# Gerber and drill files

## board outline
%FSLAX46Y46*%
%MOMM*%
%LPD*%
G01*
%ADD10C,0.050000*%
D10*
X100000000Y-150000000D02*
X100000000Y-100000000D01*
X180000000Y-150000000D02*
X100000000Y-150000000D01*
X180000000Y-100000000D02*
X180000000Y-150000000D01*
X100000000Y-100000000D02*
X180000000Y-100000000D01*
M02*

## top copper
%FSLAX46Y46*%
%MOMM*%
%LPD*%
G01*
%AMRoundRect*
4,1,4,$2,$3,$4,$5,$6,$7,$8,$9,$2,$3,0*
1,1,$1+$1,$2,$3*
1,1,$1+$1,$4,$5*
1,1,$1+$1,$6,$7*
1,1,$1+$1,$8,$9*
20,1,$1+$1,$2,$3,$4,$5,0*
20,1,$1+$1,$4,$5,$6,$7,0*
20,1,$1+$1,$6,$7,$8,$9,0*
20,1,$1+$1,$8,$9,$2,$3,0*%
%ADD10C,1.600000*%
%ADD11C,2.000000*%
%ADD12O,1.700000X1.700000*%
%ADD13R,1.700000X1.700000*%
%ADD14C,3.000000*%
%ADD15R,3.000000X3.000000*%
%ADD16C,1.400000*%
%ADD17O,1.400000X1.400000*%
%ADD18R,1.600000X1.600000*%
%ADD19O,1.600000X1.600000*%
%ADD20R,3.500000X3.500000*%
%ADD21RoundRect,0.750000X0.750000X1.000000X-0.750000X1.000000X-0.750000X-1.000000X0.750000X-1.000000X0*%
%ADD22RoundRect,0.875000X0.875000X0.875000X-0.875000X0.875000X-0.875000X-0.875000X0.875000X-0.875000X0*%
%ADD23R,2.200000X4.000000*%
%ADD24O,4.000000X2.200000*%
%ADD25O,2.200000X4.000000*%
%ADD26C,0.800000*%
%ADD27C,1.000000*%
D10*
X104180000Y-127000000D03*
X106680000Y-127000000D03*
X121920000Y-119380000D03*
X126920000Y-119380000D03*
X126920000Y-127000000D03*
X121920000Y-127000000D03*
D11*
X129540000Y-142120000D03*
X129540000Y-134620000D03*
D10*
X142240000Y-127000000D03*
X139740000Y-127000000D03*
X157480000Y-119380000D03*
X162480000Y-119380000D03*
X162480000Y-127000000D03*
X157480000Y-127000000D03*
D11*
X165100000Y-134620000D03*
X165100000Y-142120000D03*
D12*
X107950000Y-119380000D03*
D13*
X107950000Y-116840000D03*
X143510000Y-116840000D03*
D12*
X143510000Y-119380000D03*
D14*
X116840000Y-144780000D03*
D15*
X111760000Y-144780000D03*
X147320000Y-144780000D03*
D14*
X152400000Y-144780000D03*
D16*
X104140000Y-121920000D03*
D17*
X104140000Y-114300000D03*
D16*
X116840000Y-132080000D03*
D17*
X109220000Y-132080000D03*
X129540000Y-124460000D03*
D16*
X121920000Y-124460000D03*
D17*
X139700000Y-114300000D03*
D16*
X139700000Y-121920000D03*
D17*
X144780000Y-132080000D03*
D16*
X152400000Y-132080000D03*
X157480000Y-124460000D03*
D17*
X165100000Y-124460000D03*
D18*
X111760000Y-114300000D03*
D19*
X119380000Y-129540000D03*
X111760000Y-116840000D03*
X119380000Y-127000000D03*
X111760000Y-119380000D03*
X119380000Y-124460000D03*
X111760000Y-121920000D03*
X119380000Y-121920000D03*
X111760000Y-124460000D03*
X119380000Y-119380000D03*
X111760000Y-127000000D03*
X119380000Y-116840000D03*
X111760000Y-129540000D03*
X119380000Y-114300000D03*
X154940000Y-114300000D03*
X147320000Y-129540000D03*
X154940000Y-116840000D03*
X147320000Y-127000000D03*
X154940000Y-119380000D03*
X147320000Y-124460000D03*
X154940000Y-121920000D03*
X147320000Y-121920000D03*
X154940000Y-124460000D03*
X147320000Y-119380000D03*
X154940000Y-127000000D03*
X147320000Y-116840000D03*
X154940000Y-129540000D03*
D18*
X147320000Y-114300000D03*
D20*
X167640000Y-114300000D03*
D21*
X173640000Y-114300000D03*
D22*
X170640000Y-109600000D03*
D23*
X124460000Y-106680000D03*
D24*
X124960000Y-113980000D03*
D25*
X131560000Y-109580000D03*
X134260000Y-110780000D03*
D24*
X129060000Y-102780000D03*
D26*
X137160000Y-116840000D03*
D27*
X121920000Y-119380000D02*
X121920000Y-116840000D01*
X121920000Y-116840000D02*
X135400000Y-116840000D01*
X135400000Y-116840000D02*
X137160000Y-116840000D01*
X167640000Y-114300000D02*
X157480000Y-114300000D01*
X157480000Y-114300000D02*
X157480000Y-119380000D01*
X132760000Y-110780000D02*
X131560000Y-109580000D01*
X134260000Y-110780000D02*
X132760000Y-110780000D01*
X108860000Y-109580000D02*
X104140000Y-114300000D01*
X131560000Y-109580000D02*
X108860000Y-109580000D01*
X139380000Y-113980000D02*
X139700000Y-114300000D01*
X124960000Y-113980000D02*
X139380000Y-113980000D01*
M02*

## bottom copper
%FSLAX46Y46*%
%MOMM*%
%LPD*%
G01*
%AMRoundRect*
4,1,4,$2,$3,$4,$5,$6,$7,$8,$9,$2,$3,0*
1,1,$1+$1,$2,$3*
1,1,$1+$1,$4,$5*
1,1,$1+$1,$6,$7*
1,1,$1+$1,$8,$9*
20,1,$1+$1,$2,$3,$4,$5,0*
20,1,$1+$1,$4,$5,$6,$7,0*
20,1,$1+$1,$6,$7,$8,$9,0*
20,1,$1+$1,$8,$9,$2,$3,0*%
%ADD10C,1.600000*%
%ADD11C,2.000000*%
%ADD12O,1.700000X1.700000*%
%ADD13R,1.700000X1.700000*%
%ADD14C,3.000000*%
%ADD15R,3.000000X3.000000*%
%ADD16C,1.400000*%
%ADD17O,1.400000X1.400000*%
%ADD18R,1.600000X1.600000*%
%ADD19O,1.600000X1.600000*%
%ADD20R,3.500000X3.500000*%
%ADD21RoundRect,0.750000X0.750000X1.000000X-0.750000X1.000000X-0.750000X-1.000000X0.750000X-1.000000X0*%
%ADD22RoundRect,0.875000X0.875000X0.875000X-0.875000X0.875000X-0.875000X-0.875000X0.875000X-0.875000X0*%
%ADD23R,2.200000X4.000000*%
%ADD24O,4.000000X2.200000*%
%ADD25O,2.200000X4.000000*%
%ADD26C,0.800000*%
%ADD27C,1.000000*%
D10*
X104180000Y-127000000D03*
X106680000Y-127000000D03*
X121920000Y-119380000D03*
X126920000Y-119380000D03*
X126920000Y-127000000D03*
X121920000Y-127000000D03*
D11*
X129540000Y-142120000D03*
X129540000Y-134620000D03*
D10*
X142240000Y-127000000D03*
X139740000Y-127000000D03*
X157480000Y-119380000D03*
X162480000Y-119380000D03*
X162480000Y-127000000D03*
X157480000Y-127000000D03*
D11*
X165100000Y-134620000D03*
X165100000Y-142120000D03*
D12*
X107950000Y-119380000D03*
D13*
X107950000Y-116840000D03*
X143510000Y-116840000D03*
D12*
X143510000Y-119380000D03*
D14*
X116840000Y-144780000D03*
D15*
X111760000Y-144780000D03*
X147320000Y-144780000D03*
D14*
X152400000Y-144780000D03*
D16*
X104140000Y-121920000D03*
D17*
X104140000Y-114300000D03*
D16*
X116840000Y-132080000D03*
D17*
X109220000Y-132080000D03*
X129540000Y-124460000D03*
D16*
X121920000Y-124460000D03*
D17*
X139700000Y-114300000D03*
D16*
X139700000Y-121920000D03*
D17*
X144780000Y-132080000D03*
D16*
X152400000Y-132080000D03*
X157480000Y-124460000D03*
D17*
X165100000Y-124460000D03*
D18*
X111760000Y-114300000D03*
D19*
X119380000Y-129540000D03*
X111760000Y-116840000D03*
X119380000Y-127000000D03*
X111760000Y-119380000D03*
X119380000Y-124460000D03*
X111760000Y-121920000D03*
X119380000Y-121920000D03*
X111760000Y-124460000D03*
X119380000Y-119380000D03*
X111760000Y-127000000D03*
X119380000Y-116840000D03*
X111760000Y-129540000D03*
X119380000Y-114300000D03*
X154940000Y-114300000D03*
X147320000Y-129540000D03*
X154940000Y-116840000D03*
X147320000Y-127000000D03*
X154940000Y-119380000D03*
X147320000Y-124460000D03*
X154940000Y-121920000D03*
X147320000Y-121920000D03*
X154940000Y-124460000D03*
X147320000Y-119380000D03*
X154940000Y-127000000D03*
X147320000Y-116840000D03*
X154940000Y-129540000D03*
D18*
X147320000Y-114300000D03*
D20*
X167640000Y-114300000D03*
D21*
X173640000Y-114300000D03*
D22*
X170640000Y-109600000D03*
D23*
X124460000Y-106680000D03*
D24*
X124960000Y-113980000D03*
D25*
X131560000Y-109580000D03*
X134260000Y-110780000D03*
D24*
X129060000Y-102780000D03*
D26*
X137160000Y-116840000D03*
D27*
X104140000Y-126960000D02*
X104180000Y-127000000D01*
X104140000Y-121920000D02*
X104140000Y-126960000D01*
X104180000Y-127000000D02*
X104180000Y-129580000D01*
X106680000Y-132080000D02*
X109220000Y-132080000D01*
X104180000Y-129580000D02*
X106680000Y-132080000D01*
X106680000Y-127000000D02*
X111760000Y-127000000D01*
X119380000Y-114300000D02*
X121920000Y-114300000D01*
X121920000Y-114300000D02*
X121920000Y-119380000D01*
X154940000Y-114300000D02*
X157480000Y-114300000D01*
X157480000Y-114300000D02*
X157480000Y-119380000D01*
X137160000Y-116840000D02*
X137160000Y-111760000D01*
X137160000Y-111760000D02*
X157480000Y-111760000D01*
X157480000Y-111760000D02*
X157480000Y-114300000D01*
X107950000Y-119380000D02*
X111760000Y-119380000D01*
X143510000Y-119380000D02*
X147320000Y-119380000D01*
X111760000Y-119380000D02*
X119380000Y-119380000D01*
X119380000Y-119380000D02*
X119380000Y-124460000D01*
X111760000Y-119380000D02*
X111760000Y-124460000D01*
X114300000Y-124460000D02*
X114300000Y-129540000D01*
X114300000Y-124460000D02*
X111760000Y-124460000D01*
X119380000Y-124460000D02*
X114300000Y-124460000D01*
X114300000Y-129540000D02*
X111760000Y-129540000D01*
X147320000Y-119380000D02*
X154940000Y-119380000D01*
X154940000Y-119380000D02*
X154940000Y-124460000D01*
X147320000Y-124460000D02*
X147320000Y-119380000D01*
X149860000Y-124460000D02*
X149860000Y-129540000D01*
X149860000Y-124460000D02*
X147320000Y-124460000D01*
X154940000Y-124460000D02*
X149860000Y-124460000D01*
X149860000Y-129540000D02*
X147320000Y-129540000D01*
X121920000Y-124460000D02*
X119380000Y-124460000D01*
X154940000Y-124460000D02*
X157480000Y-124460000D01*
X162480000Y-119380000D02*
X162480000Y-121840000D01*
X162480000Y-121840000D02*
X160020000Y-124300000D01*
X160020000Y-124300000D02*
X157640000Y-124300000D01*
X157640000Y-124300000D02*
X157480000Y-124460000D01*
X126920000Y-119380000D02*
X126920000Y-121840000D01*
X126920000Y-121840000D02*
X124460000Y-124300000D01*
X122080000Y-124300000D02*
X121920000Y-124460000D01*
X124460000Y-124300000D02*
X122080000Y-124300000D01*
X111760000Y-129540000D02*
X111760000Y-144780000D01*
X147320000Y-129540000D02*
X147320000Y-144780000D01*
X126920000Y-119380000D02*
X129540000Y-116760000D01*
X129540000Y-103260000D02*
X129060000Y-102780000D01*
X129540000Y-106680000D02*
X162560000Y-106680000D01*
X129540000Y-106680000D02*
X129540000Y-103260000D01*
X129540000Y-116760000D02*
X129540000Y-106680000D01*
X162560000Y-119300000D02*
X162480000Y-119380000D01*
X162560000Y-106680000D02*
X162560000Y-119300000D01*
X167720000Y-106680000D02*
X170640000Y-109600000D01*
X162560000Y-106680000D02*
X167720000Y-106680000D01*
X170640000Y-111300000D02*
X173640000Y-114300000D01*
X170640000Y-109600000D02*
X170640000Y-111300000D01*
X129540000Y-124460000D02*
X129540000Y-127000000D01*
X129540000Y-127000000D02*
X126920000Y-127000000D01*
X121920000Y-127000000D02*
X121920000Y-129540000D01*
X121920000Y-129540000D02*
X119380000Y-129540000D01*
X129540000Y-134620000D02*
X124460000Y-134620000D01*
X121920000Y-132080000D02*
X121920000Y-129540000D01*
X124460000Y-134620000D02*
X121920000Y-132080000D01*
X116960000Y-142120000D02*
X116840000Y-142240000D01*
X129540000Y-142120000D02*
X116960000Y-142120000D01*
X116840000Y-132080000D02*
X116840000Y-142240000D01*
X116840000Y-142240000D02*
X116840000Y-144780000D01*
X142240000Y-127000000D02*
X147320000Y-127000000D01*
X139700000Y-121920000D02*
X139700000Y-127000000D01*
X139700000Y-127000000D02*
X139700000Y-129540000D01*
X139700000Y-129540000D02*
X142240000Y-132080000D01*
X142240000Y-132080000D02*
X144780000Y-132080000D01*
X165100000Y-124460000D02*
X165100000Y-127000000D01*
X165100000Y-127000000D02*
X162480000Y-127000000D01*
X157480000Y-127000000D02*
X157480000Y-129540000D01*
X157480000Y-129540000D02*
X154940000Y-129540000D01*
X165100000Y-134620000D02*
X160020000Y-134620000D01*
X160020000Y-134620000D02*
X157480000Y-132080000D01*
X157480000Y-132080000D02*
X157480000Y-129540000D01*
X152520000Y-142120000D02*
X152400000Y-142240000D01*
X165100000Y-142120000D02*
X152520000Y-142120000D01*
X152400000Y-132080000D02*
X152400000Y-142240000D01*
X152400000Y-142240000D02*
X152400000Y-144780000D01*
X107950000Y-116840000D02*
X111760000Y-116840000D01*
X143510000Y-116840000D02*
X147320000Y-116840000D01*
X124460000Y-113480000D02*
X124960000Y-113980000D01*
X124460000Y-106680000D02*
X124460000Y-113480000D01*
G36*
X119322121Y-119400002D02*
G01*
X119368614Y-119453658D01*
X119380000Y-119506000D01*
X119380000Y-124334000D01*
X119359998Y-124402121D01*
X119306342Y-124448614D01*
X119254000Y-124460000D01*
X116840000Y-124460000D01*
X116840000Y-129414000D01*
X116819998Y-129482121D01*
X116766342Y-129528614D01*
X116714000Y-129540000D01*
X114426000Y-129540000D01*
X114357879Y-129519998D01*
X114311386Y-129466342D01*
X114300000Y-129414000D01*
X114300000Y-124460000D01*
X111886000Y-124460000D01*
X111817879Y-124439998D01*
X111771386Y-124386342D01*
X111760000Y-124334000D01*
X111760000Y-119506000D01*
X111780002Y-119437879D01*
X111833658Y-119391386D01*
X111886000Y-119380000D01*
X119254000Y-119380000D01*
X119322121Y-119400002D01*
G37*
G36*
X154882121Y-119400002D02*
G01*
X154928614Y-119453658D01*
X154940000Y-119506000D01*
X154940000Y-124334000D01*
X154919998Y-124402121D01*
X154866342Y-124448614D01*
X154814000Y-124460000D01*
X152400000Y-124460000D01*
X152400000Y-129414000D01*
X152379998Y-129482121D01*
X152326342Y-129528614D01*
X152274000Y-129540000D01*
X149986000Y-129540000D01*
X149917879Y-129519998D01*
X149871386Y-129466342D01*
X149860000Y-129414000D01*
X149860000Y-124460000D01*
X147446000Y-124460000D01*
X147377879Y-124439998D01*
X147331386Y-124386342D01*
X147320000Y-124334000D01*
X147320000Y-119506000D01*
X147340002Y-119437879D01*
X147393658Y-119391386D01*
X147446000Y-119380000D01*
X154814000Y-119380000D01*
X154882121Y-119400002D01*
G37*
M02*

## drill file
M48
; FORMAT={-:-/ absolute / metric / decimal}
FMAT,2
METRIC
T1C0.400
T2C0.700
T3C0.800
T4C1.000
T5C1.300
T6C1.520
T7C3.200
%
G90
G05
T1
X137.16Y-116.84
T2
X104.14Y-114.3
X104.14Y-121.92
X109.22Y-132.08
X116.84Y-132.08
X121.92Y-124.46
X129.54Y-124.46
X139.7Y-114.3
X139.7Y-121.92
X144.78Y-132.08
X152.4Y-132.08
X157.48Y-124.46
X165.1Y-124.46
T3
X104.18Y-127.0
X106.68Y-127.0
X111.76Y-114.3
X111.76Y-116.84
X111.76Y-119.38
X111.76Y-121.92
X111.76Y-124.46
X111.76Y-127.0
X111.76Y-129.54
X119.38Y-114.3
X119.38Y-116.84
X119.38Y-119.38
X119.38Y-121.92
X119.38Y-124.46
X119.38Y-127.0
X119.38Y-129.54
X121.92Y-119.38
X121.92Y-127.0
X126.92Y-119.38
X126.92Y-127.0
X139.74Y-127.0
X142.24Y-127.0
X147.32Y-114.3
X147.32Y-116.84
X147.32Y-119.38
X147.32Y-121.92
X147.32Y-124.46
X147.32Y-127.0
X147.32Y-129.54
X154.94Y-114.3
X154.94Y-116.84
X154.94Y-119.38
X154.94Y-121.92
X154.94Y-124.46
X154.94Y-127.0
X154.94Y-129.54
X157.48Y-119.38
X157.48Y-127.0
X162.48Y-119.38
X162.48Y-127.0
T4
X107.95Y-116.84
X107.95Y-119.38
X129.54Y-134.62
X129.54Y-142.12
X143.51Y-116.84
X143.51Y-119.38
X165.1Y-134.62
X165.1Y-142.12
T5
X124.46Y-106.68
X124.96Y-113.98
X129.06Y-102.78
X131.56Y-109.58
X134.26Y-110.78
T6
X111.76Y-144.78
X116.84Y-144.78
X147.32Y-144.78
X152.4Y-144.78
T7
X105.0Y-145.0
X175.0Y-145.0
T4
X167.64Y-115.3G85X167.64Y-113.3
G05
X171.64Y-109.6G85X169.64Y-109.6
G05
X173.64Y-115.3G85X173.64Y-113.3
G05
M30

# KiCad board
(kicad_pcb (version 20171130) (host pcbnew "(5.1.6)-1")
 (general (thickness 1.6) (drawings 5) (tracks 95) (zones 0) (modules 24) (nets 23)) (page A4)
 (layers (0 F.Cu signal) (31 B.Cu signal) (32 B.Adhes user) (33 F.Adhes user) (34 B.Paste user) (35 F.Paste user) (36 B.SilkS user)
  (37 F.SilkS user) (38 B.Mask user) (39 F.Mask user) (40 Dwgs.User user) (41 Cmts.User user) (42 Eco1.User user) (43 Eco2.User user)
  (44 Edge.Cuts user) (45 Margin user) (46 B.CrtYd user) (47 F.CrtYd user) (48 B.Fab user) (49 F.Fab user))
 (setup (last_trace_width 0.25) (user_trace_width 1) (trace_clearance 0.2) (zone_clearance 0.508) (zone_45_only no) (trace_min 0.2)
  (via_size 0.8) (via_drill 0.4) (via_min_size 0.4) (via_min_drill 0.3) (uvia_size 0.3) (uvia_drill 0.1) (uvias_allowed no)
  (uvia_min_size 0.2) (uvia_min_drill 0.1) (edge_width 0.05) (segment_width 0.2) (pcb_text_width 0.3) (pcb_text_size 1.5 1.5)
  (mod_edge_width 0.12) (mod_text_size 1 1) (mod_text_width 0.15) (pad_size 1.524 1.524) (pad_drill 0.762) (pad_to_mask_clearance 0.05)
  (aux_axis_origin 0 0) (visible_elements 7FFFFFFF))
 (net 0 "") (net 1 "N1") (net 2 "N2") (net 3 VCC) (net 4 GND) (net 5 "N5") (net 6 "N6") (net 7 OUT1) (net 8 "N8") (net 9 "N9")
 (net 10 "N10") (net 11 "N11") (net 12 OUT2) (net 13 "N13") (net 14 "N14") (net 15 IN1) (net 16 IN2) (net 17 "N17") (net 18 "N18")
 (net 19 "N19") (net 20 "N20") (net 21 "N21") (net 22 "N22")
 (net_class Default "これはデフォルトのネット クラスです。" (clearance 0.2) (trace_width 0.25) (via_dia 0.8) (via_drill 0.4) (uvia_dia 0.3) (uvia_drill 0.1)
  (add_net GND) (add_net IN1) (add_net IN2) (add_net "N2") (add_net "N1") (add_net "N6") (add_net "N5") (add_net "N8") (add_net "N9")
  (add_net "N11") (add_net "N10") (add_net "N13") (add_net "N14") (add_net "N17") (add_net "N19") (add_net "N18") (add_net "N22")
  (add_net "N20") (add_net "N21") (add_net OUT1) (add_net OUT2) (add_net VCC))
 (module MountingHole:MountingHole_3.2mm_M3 (layer F.Cu) (at 105 145)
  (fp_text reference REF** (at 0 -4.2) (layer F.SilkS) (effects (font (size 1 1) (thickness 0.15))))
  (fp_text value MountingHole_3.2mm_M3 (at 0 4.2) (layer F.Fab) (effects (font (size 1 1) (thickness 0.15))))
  (pad 1 np_thru_hole circle (at 0 0) (size 3.2 3.2) (drill 3.2) (layers *.Cu *.Mask)))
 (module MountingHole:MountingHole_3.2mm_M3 (layer F.Cu) (at 175 145)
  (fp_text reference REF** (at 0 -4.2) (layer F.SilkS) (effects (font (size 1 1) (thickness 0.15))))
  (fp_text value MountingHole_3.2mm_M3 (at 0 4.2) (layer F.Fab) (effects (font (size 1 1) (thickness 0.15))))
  (pad 1 np_thru_hole circle (at 0 0) (size 3.2 3.2) (drill 3.2) (layers *.Cu *.Mask)))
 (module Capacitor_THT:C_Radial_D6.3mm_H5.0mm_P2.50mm (layer F.Cu) (at 106.68 127 180)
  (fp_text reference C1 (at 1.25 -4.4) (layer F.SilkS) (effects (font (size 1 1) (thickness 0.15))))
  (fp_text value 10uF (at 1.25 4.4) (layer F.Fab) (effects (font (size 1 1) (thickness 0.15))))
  (pad 2 thru_hole circle (at 2.5 0 180) (size 1.6 1.6) (drill 0.8) (layers *.Cu *.Mask) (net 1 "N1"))
  (pad 1 thru_hole circle (at 0 0 180) (size 1.6 1.6) (drill 0.8) (layers *.Cu *.Mask) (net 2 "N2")))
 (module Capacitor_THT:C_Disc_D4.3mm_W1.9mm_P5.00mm (layer F.Cu) (at 121.92 119.38)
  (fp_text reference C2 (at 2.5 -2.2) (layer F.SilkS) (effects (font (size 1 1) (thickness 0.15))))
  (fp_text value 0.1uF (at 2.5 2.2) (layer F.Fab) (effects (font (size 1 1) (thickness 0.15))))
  (pad 1 thru_hole circle (at 0 0) (size 1.6 1.6) (drill 0.8) (layers *.Cu *.Mask) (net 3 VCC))
  (pad 2 thru_hole circle (at 5 0) (size 1.6 1.6) (drill 0.8) (layers *.Cu *.Mask) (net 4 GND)))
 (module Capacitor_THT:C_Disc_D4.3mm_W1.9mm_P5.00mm (layer F.Cu) (at 121.92 127)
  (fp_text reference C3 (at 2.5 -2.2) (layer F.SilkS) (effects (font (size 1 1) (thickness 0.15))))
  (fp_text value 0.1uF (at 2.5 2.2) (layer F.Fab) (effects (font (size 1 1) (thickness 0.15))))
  (pad 2 thru_hole circle (at 5 0) (size 1.6 1.6) (drill 0.8) (layers *.Cu *.Mask) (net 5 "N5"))
  (pad 1 thru_hole circle (at 0 0) (size 1.6 1.6) (drill 0.8) (layers *.Cu *.Mask) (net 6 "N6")))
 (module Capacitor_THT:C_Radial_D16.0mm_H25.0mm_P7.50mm (layer F.Cu) (at 129.54 134.62 270)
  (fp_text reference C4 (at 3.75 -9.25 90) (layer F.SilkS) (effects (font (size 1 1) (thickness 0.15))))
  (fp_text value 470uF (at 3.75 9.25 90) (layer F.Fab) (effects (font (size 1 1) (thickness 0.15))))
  (pad 2 thru_hole circle (at 7.5 0 270) (size 2 2) (drill 1) (layers *.Cu *.Mask) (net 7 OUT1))
  (pad 1 thru_hole circle (at 0 0 270) (size 2 2) (drill 1) (layers *.Cu *.Mask) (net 6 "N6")))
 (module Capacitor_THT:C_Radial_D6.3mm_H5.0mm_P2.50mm (layer F.Cu) (at 142.24 127 180)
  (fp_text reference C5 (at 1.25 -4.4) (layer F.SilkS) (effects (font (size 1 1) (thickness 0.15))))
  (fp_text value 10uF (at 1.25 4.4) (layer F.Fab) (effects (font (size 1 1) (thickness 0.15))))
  (pad 1 thru_hole circle (at 0 0 180) (size 1.6 1.6) (drill 0.8) (layers *.Cu *.Mask) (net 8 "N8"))
  (pad 2 thru_hole circle (at 2.5 0 180) (size 1.6 1.6) (drill 0.8) (layers *.Cu *.Mask) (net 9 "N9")))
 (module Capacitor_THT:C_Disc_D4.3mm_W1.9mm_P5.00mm (layer F.Cu) (at 157.48 119.38)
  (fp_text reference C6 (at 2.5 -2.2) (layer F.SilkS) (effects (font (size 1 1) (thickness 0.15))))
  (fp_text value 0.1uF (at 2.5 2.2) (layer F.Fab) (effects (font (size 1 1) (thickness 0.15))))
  (pad 1 thru_hole circle (at 0 0) (size 1.6 1.6) (drill 0.8) (layers *.Cu *.Mask) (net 3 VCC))
  (pad 2 thru_hole circle (at 5 0) (size 1.6 1.6) (drill 0.8) (layers *.Cu *.Mask) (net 4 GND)))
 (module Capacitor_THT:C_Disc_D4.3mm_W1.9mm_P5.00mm (layer F.Cu) (at 157.48 127)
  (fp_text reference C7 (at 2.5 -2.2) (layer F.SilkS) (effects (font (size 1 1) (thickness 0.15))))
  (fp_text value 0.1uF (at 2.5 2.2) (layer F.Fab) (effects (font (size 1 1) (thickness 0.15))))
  (pad 2 thru_hole circle (at 5 0) (size 1.6 1.6) (drill 0.8) (layers *.Cu *.Mask) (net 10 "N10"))
  (pad 1 thru_hole circle (at 0 0) (size 1.6 1.6) (drill 0.8) (layers *.Cu *.Mask) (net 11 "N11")))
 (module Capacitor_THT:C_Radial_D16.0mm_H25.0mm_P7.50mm (layer F.Cu) (at 165.1 134.62 270)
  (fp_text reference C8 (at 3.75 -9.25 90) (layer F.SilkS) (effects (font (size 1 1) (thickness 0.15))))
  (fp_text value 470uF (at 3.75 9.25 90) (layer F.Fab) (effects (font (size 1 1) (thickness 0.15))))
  (pad 1 thru_hole circle (at 0 0 270) (size 2 2) (drill 1) (layers *.Cu *.Mask) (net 11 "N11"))
  (pad 2 thru_hole circle (at 7.5 0 270) (size 2 2) (drill 1) (layers *.Cu *.Mask) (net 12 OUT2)))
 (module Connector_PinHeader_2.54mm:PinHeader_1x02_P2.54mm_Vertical (layer F.Cu) (at 107.95 116.84)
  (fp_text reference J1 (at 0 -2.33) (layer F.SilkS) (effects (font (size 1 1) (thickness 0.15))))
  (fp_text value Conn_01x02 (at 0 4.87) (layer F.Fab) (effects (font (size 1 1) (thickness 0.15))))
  (pad 2 thru_hole oval (at 0 2.54) (size 1.7 1.7) (drill 1) (layers *.Cu *.Mask) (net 4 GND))
  (pad 1 thru_hole rect (at 0 0) (size 1.7 1.7) (drill 1) (layers *.Cu *.Mask) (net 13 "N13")))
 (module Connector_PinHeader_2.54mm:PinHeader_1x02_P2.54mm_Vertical (layer F.Cu) (at 143.51 116.84)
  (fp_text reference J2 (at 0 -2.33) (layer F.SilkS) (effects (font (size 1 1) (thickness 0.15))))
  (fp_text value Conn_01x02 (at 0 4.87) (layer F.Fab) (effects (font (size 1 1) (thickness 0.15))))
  (pad 1 thru_hole rect (at 0 0) (size 1.7 1.7) (drill 1) (layers *.Cu *.Mask) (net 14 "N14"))
  (pad 2 thru_hole oval (at 0 2.54) (size 1.7 1.7) (drill 1) (layers *.Cu *.Mask) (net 4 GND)))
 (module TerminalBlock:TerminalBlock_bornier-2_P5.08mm (layer F.Cu) (at 111.76 144.78)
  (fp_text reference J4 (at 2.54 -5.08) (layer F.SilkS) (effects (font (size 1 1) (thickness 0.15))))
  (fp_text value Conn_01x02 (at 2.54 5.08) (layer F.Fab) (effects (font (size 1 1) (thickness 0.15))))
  (pad 2 thru_hole circle (at 5.08 0) (size 3 3) (drill 1.52) (layers *.Cu *.Mask) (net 7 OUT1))
  (pad 1 thru_hole rect (at 0 0) (size 3 3) (drill 1.52) (layers *.Cu *.Mask) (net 4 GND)))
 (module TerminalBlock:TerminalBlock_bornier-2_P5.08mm (layer F.Cu) (at 147.32 144.78)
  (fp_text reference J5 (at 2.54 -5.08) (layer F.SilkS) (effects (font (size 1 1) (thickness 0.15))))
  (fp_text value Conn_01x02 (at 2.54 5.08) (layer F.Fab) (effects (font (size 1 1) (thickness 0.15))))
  (pad 1 thru_hole rect (at 0 0) (size 3 3) (drill 1.52) (layers *.Cu *.Mask) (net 4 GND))
  (pad 2 thru_hole circle (at 5.08 0) (size 3 3) (drill 1.52) (layers *.Cu *.Mask) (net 12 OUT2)))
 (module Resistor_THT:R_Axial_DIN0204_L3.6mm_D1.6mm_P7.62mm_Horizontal (layer F.Cu) (at 104.14 121.92 90)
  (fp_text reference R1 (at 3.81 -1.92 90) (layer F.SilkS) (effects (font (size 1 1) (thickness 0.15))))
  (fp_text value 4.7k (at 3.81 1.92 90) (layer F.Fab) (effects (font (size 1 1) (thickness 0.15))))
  (pad 1 thru_hole circle (at 0 0 90) (size 1.4 1.4) (drill 0.7) (layers *.Cu *.Mask) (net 1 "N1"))
  (pad 2 thru_hole oval (at 7.62 0 90) (size 1.4 1.4) (drill 0.7) (layers *.Cu *.Mask) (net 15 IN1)))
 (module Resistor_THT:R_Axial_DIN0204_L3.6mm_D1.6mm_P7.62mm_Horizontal (layer F.Cu) (at 116.84 132.08 180)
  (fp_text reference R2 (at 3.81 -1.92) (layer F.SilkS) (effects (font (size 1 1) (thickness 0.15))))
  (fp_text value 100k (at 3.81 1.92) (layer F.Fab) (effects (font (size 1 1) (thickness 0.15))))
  (pad 1 thru_hole circle (at 0 0 180) (size 1.4 1.4) (drill 0.7) (layers *.Cu *.Mask) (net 7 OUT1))
  (pad 2 thru_hole oval (at 7.62 0 180) (size 1.4 1.4) (drill 0.7) (layers *.Cu *.Mask) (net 1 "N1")))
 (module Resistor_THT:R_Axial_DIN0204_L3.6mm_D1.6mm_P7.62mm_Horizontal (layer F.Cu) (at 121.92 124.46)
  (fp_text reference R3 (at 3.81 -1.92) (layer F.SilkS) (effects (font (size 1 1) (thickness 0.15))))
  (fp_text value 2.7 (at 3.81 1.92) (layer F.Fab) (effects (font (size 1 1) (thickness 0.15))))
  (pad 2 thru_hole oval (at 7.62 0) (size 1.4 1.4) (drill 0.7) (layers *.Cu *.Mask) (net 5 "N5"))
  (pad 1 thru_hole circle (at 0 0) (size 1.4 1.4) (drill 0.7) (layers *.Cu *.Mask) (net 4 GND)))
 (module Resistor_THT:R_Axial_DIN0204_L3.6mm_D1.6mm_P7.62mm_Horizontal (layer F.Cu) (at 139.7 121.92 90)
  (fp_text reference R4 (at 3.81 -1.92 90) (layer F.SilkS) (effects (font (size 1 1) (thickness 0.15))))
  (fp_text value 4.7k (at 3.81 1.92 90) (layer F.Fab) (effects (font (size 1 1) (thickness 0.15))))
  (pad 2 thru_hole oval (at 7.62 0 90) (size 1.4 1.4) (drill 0.7) (layers *.Cu *.Mask) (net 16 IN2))
  (pad 1 thru_hole circle (at 0 0 90) (size 1.4 1.4) (drill 0.7) (layers *.Cu *.Mask) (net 9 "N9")))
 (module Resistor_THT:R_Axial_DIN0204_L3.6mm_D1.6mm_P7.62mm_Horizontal (layer F.Cu) (at 152.4 132.08 180)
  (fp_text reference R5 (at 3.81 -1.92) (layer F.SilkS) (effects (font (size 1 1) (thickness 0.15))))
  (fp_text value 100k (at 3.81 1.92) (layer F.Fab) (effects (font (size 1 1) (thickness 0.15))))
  (pad 2 thru_hole oval (at 7.62 0 180) (size 1.4 1.4) (drill 0.7) (layers *.Cu *.Mask) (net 9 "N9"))
  (pad 1 thru_hole circle (at 0 0 180) (size 1.4 1.4) (drill 0.7) (layers *.Cu *.Mask) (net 12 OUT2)))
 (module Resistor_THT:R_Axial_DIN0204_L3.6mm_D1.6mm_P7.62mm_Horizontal (layer F.Cu) (at 157.48 124.46)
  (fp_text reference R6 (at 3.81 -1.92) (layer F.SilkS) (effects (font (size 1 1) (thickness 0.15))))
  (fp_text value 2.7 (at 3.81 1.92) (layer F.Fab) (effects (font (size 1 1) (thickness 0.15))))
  (pad 1 thru_hole circle (at 0 0) (size 1.4 1.4) (drill 0.7) (layers *.Cu *.Mask) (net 4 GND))
  (pad 2 thru_hole oval (at 7.62 0) (size 1.4 1.4) (drill 0.7) (layers *.Cu *.Mask) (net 10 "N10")))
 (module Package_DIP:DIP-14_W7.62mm (layer F.Cu) (at 111.76 114.3)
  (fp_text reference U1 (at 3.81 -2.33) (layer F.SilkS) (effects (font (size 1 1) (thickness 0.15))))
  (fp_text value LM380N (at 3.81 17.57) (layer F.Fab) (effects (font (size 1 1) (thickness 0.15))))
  (pad 1 thru_hole rect (at 0 0) (size 1.6 1.6) (drill 0.8) (layers *.Cu *.Mask) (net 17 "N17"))
  (pad 8 thru_hole oval (at 7.62 15.24) (size 1.6 1.6) (drill 0.8) (layers *.Cu *.Mask) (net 6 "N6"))
  (pad 2 thru_hole oval (at 0 2.54) (size 1.6 1.6) (drill 0.8) (layers *.Cu *.Mask) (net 13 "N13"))
  (pad 9 thru_hole oval (at 7.62 12.7) (size 1.6 1.6) (drill 0.8) (layers *.Cu *.Mask) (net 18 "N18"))
  (pad 3 thru_hole oval (at 0 5.08) (size 1.6 1.6) (drill 0.8) (layers *.Cu *.Mask) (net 4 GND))
  (pad 10 thru_hole oval (at 7.62 10.16) (size 1.6 1.6) (drill 0.8) (layers *.Cu *.Mask) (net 4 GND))
  (pad 4 thru_hole oval (at 0 7.62) (size 1.6 1.6) (drill 0.8) (layers *.Cu *.Mask) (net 4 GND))
  (pad 11 thru_hole oval (at 7.62 7.62) (size 1.6 1.6) (drill 0.8) (layers *.Cu *.Mask) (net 4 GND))
  (pad 5 thru_hole oval (at 0 10.16) (size 1.6 1.6) (drill 0.8) (layers *.Cu *.Mask) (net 4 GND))
  (pad 12 thru_hole oval (at 7.62 5.08) (size 1.6 1.6) (drill 0.8) (layers *.Cu *.Mask) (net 4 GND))
  (pad 6 thru_hole oval (at 0 12.7) (size 1.6 1.6) (drill 0.8) (layers *.Cu *.Mask) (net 2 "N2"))
  (pad 13 thru_hole oval (at 7.62 2.54) (size 1.6 1.6) (drill 0.8) (layers *.Cu *.Mask) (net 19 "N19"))
  (pad 7 thru_hole oval (at 0 15.24) (size 1.6 1.6) (drill 0.8) (layers *.Cu *.Mask) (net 4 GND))
  (pad 14 thru_hole oval (at 7.62 0) (size 1.6 1.6) (drill 0.8) (layers *.Cu *.Mask) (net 3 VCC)))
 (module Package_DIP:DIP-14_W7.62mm (layer F.Cu) (at 147.32 114.3)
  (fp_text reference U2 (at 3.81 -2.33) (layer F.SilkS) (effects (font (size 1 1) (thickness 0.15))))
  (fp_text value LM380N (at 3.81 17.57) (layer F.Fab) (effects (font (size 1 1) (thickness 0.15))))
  (pad 14 thru_hole oval (at 7.62 0) (size 1.6 1.6) (drill 0.8) (layers *.Cu *.Mask) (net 3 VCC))
  (pad 7 thru_hole oval (at 0 15.24) (size 1.6 1.6) (drill 0.8) (layers *.Cu *.Mask) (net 4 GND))
  (pad 13 thru_hole oval (at 7.62 2.54) (size 1.6 1.6) (drill 0.8) (layers *.Cu *.Mask) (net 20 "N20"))
  (pad 6 thru_hole oval (at 0 12.7) (size 1.6 1.6) (drill 0.8) (layers *.Cu *.Mask) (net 8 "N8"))
  (pad 12 thru_hole oval (at 7.62 5.08) (size 1.6 1.6) (drill 0.8) (layers *.Cu *.Mask) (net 4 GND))
  (pad 5 thru_hole oval (at 0 10.16) (size 1.6 1.6) (drill 0.8) (layers *.Cu *.Mask) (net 4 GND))
  (pad 11 thru_hole oval (at 7.62 7.62) (size 1.6 1.6) (drill 0.8) (layers *.Cu *.Mask) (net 4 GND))
  (pad 4 thru_hole oval (at 0 7.62) (size 1.6 1.6) (drill 0.8) (layers *.Cu *.Mask) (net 4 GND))
  (pad 10 thru_hole oval (at 7.62 10.16) (size 1.6 1.6) (drill 0.8) (layers *.Cu *.Mask) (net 4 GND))
  (pad 3 thru_hole oval (at 0 5.08) (size 1.6 1.6) (drill 0.8) (layers *.Cu *.Mask) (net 4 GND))
  (pad 9 thru_hole oval (at 7.62 12.7) (size 1.6 1.6) (drill 0.8) (layers *.Cu *.Mask) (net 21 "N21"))
  (pad 2 thru_hole oval (at 0 2.54) (size 1.6 1.6) (drill 0.8) (layers *.Cu *.Mask) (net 14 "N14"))
  (pad 8 thru_hole oval (at 7.62 15.24) (size 1.6 1.6) (drill 0.8) (layers *.Cu *.Mask) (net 11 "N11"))
  (pad 1 thru_hole rect (at 0 0) (size 1.6 1.6) (drill 0.8) (layers *.Cu *.Mask) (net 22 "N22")))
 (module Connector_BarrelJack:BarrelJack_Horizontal (layer F.Cu) (at 167.64 114.3 180)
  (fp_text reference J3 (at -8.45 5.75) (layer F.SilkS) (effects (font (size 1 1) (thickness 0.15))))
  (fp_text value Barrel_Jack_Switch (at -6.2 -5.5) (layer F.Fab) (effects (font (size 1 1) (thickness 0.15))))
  (pad 1 thru_hole rect (at 0 0 180) (size 3.5 3.5) (drill oval 1 3) (layers *.Cu *.Mask) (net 3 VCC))
  (pad 2 thru_hole roundrect (at -6 0 180) (size 3 3.5) (drill oval 1 3) (layers *.Cu *.Mask) (roundrect_rratio 0.25) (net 4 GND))
  (pad 3 thru_hole roundrect (at -3 4.7 180) (size 3.5 3.5) (drill oval 3 1) (layers *.Cu *.Mask) (roundrect_rratio 0.25) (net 4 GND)))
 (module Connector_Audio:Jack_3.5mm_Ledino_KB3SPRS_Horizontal (layer F.Cu) (at 124.46 106.68 270)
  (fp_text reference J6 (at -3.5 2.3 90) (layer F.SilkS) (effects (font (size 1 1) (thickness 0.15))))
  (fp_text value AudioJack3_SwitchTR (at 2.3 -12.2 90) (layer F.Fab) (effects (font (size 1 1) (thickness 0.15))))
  (pad T thru_hole rect (at 0 0 270) (size 4 2.2) (drill 1.3) (layers *.Cu *.Mask) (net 16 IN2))
  (pad TN thru_hole oval (at 7.3 -0.5) (size 4 2.2) (drill 1.3) (layers *.Cu *.Mask) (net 16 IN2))
  (pad RN thru_hole oval (at 2.9 -7.1 270) (size 4 2.2) (drill 1.3) (layers *.Cu *.Mask) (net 15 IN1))
  (pad R thru_hole oval (at 4.1 -9.8 270) (size 4 2.2) (drill 1.3) (layers *.Cu *.Mask) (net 15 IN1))
  (pad S thru_hole oval (at -3.9 -4.6 270) (size 2.2 4) (drill 1.3) (layers *.Cu *.Mask) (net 4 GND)))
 (gr_line (start 100 150) (end 100 100) (layer Edge.Cuts) (width 0.05))
 (gr_line (start 180 150) (end 100 150) (layer Edge.Cuts) (width 0.05))
 (gr_line (start 180 100) (end 180 150) (layer Edge.Cuts) (width 0.05))
 (gr_line (start 100 100) (end 180 100) (layer Edge.Cuts) (width 0.05))
 (segment (start 104.14 126.96) (end 104.18 127) (width 1) (layer B.Cu) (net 1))
 (segment (start 104.14 121.92) (end 104.14 126.96) (width 1) (layer B.Cu) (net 1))
 (segment (start 104.18 127) (end 104.18 129.58) (width 1) (layer B.Cu) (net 1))
 (segment (start 106.68 132.08) (end 109.22 132.08) (width 1) (layer B.Cu) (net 1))
 (segment (start 104.18 129.58) (end 106.68 132.08) (width 1) (layer B.Cu) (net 1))
 (segment (start 106.68 127) (end 111.76 127) (width 1) (layer B.Cu) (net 2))
 (segment (start 119.38 114.3) (end 121.92 114.3) (width 1) (layer B.Cu) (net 3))
 (segment (start 121.92 114.3) (end 121.92 119.38) (width 1) (layer B.Cu) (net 3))
 (segment (start 154.94 114.3) (end 157.48 114.3) (width 1) (layer B.Cu) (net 3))
 (segment (start 157.48 114.3) (end 157.48 119.38) (width 1) (layer B.Cu) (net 3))
 (segment (start 121.92 119.38) (end 121.92 116.84) (width 1) (layer F.Cu) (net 3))
 (via (at 137.16 116.84) (size 0.8) (drill 0.4) (layers F.Cu B.Cu) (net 3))
 (segment (start 121.92 116.84) (end 135.4 116.84) (width 1) (layer F.Cu) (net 3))
 (segment (start 135.4 116.84) (end 137.16 116.84) (width 1) (layer F.Cu) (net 3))
 (segment (start 137.16 116.84) (end 137.16 111.76) (width 1) (layer B.Cu) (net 3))
 (segment (start 137.16 111.76) (end 157.48 111.76) (width 1) (layer B.Cu) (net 3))
 (segment (start 157.48 111.76) (end 157.48 114.3) (width 1) (layer B.Cu) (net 3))
 (segment (start 167.64 114.3) (end 157.48 114.3) (width 1) (layer F.Cu) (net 3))
 (segment (start 157.48 114.3) (end 157.48 119.38) (width 1) (layer F.Cu) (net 3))
 (segment (start 107.95 119.38) (end 111.76 119.38) (width 1) (layer B.Cu) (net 4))
 (segment (start 143.51 119.38) (end 147.32 119.38) (width 1) (layer B.Cu) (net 4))
 (segment (start 111.76 119.38) (end 119.38 119.38) (width 1) (layer B.Cu) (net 4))
 (segment (start 119.38 119.38) (end 119.38 124.46) (width 1) (layer B.Cu) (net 4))
 (segment (start 111.76 119.38) (end 111.76 124.46) (width 1) (layer B.Cu) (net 4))
 (segment (start 114.3 124.46) (end 114.3 129.54) (width 1) (layer B.Cu) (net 4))
 (segment (start 114.3 124.46) (end 111.76 124.46) (width 1) (layer B.Cu) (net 4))
 (segment (start 119.38 124.46) (end 114.3 124.46) (width 1) (layer B.Cu) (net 4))
 (segment (start 114.3 129.54) (end 111.76 129.54) (width 1) (layer B.Cu) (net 4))
 (segment (start 147.32 119.38) (end 154.94 119.38) (width 1) (layer B.Cu) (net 4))
 (segment (start 154.94 119.38) (end 154.94 124.46) (width 1) (layer B.Cu) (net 4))
 (segment (start 147.32 124.46) (end 147.32 119.38) (width 1) (layer B.Cu) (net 4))
 (segment (start 149.86 124.46) (end 149.86 129.54) (width 1) (layer B.Cu) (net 4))
 (segment (start 149.86 124.46) (end 147.32 124.46) (width 1) (layer B.Cu) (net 4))
 (segment (start 154.94 124.46) (end 149.86 124.46) (width 1) (layer B.Cu) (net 4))
 (segment (start 149.86 129.54) (end 147.32 129.54) (width 1) (layer B.Cu) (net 4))
 (segment (start 121.92 124.46) (end 119.38 124.46) (width 1) (layer B.Cu) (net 4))
 (segment (start 154.94 124.46) (end 157.48 124.46) (width 1) (layer B.Cu) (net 4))
 (segment (start 162.48 119.38) (end 162.48 121.84) (width 1) (layer B.Cu) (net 4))
 (segment (start 162.48 121.84) (end 160.02 124.3) (width 1) (layer B.Cu) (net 4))
 (segment (start 160.02 124.3) (end 157.64 124.3) (width 1) (layer B.Cu) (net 4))
 (segment (start 157.64 124.3) (end 157.48 124.46) (width 1) (layer B.Cu) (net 4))
 (segment (start 126.92 119.38) (end 126.92 121.84) (width 1) (layer B.Cu) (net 4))
 (segment (start 126.92 121.84) (end 124.46 124.3) (width 1) (layer B.Cu) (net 4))
 (segment (start 122.08 124.3) (end 121.92 124.46) (width 1) (layer B.Cu) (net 4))
 (segment (start 124.46 124.3) (end 122.08 124.3) (width 1) (layer B.Cu) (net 4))
 (segment (start 111.76 129.54) (end 111.76 144.78) (width 1) (layer B.Cu) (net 4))
 (segment (start 147.32 129.54) (end 147.32 144.78) (width 1) (layer B.Cu) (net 4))
 (segment (start 126.92 119.38) (end 129.54 116.76) (width 1) (layer B.Cu) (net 4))
 (segment (start 129.54 103.26) (end 129.06 102.78) (width 1) (layer B.Cu) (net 4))
 (segment (start 129.54 106.68) (end 162.56 106.68) (width 1) (layer B.Cu) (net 4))
 (segment (start 129.54 106.68) (end 129.54 103.26) (width 1) (layer B.Cu) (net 4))
 (segment (start 129.54 116.76) (end 129.54 106.68) (width 1) (layer B.Cu) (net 4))
 (segment (start 162.56 119.3) (end 162.48 119.38) (width 1) (layer B.Cu) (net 4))
 (segment (start 162.56 106.68) (end 162.56 119.3) (width 1) (layer B.Cu) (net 4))
 (segment (start 167.72 106.68) (end 170.64 109.6) (width 1) (layer B.Cu) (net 4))
 (segment (start 162.56 106.68) (end 167.72 106.68) (width 1) (layer B.Cu) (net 4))
 (segment (start 170.64 111.3) (end 173.64 114.3) (width 1) (layer B.Cu) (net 4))
 (segment (start 170.64 109.6) (end 170.64 111.3) (width 1) (layer B.Cu) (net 4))
 (segment (start 129.54 124.46) (end 129.54 127) (width 1) (layer B.Cu) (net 5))
 (segment (start 129.54 127) (end 126.92 127) (width 1) (layer B.Cu) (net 5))
 (segment (start 121.92 127) (end 121.92 129.54) (width 1) (layer B.Cu) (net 6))
 (segment (start 121.92 129.54) (end 119.38 129.54) (width 1) (layer B.Cu) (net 6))
 (segment (start 129.54 134.62) (end 124.46 134.62) (width 1) (layer B.Cu) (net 6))
 (segment (start 121.92 132.08) (end 121.92 129.54) (width 1) (layer B.Cu) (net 6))
 (segment (start 124.46 134.62) (end 121.92 132.08) (width 1) (layer B.Cu) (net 6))
 (segment (start 116.96 142.12) (end 116.84 142.24) (width 1) (layer B.Cu) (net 7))
 (segment (start 129.54 142.12) (end 116.96 142.12) (width 1) (layer B.Cu) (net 7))
 (segment (start 116.84 132.08) (end 116.84 142.24) (width 1) (layer B.Cu) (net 7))
 (segment (start 116.84 142.24) (end 116.84 144.78) (width 1) (layer B.Cu) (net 7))
 (segment (start 142.24 127) (end 147.32 127) (width 1) (layer B.Cu) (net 8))
 (segment (start 139.7 121.92) (end 139.7 127) (width 1) (layer B.Cu) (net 9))
 (segment (start 139.7 127) (end 139.7 129.54) (width 1) (layer B.Cu) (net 9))
 (segment (start 139.7 129.54) (end 142.24 132.08) (width 1) (layer B.Cu) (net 9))
 (segment (start 142.24 132.08) (end 144.78 132.08) (width 1) (layer B.Cu) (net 9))
 (segment (start 165.1 124.46) (end 165.1 127) (width 1) (layer B.Cu) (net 10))
 (segment (start 165.1 127) (end 162.48 127) (width 1) (layer B.Cu) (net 10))
 (segment (start 157.48 127) (end 157.48 129.54) (width 1) (layer B.Cu) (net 11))
 (segment (start 157.48 129.54) (end 154.94 129.54) (width 1) (layer B.Cu) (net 11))
 (segment (start 165.1 134.62) (end 160.02 134.62) (width 1) (layer B.Cu) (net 11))
 (segment (start 160.02 134.62) (end 157.48 132.08) (width 1) (layer B.Cu) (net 11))
 (segment (start 157.48 132.08) (end 157.48 129.54) (width 1) (layer B.Cu) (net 11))
 (segment (start 152.52 142.12) (end 152.4 142.24) (width 1) (layer B.Cu) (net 12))
 (segment (start 165.1 142.12) (end 152.52 142.12) (width 1) (layer B.Cu) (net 12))
 (segment (start 152.4 132.08) (end 152.4 142.24) (width 1) (layer B.Cu) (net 12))
 (segment (start 152.4 142.24) (end 152.4 144.78) (width 1) (layer B.Cu) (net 12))
 (segment (start 107.95 116.84) (end 111.76 116.84) (width 1) (layer B.Cu) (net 13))
 (segment (start 143.51 116.84) (end 147.32 116.84) (width 1) (layer B.Cu) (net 14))
 (segment (start 132.76 110.78) (end 131.56 109.58) (width 1) (layer F.Cu) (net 15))
 (segment (start 134.26 110.78) (end 132.76 110.78) (width 1) (layer F.Cu) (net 15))
 (segment (start 108.86 109.58) (end 104.14 114.3) (width 1) (layer F.Cu) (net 15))
 (segment (start 131.56 109.58) (end 108.86 109.58) (width 1) (layer F.Cu) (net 15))
 (segment (start 124.46 113.48) (end 124.96 113.98) (width 1) (layer B.Cu) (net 16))
 (segment (start 124.46 106.68) (end 124.46 113.48) (width 1) (layer B.Cu) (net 16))
 (segment (start 139.38 113.98) (end 139.7 114.3) (width 1) (layer F.Cu) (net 16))
 (segment (start 124.96 113.98) (end 139.38 113.98) (width 1) (layer F.Cu) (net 16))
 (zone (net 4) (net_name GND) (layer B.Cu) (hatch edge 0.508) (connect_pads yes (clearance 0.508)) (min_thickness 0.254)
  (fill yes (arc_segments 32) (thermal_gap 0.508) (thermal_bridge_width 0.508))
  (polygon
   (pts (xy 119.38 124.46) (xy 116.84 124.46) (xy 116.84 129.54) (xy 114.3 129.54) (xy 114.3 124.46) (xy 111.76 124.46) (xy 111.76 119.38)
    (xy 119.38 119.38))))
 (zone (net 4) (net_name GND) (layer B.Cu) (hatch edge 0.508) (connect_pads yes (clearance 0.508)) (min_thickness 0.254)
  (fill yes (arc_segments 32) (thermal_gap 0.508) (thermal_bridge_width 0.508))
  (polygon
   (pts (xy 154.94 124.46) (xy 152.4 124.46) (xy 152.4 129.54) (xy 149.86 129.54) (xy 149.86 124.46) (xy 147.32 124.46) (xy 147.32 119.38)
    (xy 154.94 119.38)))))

